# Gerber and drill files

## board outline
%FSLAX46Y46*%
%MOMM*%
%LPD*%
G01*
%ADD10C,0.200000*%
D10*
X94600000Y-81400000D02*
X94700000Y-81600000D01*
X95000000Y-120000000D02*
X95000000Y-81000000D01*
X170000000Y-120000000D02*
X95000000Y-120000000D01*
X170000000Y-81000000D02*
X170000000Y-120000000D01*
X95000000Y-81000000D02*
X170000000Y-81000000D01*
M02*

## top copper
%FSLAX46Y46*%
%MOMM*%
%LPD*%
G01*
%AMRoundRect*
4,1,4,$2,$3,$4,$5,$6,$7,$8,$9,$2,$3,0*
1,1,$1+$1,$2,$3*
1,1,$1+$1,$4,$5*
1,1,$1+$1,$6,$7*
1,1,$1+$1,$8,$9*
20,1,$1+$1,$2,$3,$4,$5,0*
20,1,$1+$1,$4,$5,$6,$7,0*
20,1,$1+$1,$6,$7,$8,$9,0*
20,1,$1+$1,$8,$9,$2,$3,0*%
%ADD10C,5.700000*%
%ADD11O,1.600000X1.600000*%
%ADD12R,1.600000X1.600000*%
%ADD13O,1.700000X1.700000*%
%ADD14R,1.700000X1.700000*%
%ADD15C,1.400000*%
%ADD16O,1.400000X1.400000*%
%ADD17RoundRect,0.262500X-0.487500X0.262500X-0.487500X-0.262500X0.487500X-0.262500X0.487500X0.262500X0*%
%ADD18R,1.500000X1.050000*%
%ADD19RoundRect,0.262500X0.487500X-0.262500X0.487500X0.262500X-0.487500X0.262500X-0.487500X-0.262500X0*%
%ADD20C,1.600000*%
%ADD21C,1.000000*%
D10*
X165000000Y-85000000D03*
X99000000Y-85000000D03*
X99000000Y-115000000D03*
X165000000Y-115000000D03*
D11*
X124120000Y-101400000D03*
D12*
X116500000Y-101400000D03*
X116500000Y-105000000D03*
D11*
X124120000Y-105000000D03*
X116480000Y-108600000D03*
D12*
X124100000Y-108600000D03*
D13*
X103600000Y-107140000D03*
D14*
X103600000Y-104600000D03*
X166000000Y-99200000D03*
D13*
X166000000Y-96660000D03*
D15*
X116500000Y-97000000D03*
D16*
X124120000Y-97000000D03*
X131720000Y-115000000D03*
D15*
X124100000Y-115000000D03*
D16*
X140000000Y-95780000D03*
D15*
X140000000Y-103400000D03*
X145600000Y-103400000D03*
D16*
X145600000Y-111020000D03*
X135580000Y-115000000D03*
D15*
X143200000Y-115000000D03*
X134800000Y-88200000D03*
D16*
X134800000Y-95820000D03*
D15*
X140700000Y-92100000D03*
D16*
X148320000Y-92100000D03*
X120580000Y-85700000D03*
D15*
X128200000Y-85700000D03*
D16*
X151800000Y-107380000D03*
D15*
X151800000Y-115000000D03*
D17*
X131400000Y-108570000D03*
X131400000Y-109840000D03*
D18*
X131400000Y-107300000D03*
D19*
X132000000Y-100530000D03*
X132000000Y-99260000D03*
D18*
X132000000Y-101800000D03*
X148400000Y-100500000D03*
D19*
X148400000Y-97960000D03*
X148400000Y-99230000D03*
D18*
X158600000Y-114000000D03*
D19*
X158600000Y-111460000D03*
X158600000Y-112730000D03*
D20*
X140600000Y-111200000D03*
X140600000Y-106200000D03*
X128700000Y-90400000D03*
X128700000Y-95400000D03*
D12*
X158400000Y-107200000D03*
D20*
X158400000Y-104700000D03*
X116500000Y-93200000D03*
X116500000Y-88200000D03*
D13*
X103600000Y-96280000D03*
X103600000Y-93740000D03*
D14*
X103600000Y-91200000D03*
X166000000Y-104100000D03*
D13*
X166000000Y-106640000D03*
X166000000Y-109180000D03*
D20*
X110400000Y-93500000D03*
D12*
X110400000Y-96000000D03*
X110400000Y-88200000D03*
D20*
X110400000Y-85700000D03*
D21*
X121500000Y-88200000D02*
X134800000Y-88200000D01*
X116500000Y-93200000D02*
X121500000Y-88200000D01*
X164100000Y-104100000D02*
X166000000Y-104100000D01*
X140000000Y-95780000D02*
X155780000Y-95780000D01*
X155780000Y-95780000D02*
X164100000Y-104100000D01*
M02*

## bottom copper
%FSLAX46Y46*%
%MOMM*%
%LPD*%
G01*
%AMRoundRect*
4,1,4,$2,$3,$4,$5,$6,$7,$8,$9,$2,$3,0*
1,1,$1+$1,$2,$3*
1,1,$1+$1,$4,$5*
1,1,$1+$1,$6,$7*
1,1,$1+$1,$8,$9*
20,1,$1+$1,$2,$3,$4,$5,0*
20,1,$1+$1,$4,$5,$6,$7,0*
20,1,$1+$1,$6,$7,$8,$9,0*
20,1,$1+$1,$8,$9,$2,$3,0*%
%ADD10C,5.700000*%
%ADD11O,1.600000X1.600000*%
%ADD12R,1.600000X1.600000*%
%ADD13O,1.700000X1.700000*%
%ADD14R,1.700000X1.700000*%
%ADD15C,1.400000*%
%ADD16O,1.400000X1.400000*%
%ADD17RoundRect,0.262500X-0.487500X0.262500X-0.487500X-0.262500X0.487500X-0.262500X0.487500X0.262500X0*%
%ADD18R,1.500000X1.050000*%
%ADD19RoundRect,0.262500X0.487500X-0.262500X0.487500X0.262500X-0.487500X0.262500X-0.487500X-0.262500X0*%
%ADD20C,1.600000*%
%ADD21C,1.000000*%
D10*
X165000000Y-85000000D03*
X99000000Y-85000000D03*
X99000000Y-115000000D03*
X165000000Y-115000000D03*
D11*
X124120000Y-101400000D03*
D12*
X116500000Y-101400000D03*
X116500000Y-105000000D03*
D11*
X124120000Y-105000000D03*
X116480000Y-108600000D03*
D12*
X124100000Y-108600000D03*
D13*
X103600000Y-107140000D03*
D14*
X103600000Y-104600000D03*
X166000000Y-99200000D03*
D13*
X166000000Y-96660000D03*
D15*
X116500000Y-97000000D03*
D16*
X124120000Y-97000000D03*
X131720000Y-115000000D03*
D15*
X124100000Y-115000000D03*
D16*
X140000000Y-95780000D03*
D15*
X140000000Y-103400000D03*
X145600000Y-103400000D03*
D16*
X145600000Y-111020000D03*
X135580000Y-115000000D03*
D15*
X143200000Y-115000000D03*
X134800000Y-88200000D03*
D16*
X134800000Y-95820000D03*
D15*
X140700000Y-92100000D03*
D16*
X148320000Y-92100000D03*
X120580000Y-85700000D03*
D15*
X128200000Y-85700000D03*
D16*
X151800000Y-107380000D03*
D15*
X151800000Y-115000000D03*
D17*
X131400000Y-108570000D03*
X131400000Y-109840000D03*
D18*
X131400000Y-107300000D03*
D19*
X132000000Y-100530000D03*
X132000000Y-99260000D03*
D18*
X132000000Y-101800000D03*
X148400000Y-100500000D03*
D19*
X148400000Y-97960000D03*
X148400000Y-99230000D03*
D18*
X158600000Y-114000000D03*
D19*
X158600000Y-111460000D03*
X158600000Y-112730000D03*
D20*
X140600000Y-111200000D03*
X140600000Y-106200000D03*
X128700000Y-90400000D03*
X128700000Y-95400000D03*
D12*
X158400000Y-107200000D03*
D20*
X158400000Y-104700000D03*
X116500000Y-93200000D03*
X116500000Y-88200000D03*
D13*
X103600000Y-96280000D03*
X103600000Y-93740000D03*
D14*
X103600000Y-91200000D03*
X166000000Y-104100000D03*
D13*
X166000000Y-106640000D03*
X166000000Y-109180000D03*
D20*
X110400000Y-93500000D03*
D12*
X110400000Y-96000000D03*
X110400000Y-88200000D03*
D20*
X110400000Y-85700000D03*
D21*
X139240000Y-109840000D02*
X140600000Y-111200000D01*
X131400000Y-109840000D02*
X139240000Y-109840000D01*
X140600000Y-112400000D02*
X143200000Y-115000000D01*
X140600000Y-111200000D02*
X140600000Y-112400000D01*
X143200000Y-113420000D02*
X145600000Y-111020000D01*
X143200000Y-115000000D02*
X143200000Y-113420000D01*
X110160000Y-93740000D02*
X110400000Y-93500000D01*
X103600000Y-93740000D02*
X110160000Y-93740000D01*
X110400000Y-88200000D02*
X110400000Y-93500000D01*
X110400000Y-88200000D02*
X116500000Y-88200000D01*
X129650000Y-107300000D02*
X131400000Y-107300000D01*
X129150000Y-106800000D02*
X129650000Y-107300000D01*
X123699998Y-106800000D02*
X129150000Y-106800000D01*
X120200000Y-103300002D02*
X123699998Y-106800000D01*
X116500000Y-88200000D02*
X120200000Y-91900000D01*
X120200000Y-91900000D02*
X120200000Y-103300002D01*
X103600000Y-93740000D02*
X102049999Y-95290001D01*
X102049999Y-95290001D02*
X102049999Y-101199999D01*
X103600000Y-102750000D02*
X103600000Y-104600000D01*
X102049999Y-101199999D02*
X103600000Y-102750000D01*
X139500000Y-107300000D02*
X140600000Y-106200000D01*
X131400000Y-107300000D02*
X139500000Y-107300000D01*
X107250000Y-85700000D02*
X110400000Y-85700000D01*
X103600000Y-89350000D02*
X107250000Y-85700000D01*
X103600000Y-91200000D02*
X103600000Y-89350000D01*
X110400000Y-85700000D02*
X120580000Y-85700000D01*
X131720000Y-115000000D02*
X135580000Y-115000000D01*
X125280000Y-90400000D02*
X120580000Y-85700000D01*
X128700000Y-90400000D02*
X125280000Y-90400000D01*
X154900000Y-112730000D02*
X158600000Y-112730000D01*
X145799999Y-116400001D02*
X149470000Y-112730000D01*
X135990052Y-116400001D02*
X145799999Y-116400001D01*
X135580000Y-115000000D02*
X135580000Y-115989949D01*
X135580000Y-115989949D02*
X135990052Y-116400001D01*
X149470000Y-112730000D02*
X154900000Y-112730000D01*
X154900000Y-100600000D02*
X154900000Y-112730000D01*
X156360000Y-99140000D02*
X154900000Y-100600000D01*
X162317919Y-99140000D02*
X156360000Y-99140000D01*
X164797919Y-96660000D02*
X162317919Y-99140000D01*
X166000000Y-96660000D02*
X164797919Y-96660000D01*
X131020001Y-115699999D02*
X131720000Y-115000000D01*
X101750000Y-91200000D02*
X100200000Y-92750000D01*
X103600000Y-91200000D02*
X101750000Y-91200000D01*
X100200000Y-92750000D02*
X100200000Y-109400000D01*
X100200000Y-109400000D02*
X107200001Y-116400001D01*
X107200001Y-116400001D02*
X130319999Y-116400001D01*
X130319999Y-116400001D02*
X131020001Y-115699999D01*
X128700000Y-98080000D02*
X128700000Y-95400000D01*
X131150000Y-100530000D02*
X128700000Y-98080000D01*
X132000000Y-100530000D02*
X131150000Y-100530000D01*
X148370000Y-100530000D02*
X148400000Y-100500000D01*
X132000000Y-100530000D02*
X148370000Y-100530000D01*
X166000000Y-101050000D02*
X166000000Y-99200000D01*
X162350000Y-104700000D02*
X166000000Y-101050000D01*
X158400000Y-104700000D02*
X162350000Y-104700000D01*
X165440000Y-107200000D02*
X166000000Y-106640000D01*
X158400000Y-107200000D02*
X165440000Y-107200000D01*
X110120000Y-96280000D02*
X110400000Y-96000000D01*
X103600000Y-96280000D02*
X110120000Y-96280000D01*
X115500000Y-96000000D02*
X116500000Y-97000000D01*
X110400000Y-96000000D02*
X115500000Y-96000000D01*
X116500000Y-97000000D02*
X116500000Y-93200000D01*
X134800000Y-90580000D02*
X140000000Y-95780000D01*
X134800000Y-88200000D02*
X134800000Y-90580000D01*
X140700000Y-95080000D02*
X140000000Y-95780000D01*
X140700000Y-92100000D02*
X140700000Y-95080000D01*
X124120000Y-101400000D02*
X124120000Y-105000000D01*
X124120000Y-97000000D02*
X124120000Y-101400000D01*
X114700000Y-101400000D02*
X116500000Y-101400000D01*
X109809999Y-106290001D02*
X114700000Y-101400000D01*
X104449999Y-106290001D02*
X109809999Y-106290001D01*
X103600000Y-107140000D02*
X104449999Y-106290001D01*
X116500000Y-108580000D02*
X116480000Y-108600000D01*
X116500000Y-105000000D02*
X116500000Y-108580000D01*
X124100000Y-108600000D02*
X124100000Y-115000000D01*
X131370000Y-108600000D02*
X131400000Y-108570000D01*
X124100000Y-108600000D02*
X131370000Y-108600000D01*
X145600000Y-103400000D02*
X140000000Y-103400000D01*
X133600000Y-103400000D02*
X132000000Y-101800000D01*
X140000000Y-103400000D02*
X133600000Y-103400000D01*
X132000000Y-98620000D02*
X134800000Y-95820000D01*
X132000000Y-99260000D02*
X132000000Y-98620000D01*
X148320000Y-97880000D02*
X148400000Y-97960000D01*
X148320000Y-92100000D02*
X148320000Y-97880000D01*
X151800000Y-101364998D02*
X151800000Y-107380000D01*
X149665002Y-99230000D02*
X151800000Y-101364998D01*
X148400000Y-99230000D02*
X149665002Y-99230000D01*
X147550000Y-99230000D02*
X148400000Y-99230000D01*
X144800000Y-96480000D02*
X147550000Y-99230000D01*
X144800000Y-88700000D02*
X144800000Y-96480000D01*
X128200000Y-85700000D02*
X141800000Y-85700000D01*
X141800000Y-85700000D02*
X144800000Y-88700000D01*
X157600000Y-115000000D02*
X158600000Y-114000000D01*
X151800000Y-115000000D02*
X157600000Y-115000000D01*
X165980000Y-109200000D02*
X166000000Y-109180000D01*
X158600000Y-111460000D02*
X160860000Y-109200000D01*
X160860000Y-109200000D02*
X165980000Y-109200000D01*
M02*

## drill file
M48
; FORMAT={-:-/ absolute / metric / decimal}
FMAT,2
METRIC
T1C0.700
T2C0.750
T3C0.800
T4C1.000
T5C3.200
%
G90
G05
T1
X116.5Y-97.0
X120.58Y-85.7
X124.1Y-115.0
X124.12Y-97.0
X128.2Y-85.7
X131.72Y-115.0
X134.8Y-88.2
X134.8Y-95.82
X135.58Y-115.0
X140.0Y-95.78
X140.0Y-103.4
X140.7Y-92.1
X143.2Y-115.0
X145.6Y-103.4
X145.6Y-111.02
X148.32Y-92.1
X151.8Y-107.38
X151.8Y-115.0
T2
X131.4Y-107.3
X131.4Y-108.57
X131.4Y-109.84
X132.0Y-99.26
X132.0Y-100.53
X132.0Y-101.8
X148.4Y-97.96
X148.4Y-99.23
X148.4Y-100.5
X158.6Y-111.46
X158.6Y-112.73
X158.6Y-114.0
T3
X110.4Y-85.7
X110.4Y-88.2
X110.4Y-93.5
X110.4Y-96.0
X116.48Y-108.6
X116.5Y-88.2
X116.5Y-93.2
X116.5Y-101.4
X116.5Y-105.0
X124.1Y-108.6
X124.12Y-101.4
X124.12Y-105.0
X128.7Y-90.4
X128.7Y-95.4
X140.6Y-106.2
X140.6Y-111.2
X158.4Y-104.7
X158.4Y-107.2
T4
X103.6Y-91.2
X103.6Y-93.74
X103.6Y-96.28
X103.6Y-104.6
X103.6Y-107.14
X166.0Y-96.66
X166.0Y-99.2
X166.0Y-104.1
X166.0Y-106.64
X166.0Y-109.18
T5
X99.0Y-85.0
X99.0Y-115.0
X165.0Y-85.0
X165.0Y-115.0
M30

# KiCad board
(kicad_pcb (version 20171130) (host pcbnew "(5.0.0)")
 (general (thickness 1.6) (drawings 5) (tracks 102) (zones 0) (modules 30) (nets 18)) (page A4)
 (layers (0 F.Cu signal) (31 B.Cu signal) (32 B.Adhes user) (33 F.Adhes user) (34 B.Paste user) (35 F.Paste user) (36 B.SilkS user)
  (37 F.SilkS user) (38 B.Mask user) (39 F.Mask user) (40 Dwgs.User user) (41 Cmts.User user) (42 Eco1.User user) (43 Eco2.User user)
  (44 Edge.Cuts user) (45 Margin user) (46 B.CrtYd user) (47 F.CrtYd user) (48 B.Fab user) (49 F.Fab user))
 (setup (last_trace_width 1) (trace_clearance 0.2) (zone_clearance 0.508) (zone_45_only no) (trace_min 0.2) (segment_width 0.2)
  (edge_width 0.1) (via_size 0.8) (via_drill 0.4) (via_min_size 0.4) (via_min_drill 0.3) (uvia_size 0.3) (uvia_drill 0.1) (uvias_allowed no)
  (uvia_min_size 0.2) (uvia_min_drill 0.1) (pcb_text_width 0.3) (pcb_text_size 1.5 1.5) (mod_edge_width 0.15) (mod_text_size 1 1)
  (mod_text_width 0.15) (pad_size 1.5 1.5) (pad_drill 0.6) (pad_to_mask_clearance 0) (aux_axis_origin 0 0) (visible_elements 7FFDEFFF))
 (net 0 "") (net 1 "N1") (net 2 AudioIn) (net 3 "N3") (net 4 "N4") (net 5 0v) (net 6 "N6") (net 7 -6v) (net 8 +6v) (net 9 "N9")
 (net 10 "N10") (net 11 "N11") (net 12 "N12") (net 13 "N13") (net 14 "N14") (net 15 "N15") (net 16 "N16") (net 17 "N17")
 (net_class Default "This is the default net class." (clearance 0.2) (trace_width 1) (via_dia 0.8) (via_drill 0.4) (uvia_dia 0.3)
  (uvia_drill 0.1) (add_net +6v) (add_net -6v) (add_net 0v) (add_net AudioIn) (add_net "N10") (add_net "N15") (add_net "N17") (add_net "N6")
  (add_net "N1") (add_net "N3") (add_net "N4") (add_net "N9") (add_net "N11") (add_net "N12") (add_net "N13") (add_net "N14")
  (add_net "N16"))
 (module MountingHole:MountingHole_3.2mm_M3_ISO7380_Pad (layer F.Cu) (at 165 85)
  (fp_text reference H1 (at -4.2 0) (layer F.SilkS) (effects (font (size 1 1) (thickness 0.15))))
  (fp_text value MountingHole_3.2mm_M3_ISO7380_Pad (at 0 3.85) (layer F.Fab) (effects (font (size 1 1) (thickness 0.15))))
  (pad 1 thru_hole circle (at 0 0) (size 5.7 5.7) (drill 3.2) (layers *.Cu *.Mask)))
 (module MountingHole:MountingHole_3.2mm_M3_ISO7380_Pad (layer F.Cu) (at 99 85)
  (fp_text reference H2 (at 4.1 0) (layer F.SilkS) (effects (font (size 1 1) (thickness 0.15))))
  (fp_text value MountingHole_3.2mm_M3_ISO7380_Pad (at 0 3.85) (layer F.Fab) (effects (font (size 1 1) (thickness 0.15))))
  (pad 1 thru_hole circle (at 0 0) (size 5.7 5.7) (drill 3.2) (layers *.Cu *.Mask)))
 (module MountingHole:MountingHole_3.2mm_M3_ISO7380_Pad (layer F.Cu) (at 99 115)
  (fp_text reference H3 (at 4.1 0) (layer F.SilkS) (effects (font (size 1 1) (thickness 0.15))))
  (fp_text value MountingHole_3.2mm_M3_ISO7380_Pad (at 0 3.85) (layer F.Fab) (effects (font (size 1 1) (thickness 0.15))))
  (pad 1 thru_hole circle (at 0 0) (size 5.7 5.7) (drill 3.2) (layers *.Cu *.Mask)))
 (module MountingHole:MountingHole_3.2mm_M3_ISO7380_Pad (layer F.Cu) (at 165 115)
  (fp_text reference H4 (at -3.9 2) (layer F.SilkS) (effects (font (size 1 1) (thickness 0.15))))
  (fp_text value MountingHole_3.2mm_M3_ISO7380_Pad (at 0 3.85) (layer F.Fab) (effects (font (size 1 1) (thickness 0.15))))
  (pad 1 thru_hole circle (at 0 0) (size 5.7 5.7) (drill 3.2) (layers *.Cu *.Mask)))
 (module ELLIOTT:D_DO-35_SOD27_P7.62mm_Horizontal (layer F.Cu) (at 116.5 101.4)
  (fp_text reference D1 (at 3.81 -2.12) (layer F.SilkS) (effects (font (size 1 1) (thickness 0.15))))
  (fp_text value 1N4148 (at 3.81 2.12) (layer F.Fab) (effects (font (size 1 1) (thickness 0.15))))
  (pad 2 thru_hole oval (at 7.62 0) (size 1.6 1.6) (drill 0.8) (layers *.Cu *.Mask) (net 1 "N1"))
  (pad 1 thru_hole rect (at 0 0) (size 1.6 1.6) (drill 0.8) (layers *.Cu *.Mask) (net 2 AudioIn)))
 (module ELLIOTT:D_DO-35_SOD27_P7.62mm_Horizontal (layer F.Cu) (at 116.5 105)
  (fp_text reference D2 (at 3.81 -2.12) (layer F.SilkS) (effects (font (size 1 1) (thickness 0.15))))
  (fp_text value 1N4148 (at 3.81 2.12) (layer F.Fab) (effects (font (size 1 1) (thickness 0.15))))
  (pad 1 thru_hole rect (at 0 0) (size 1.6 1.6) (drill 0.8) (layers *.Cu *.Mask) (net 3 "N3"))
  (pad 2 thru_hole oval (at 7.62 0) (size 1.6 1.6) (drill 0.8) (layers *.Cu *.Mask) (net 1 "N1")))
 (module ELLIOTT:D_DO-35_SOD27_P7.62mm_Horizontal (layer F.Cu) (at 124.1 108.6 180)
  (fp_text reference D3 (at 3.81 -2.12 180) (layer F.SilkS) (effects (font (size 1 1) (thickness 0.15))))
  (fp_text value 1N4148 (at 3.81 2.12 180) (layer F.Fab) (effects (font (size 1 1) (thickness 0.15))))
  (pad 2 thru_hole oval (at 7.62 0 180) (size 1.6 1.6) (drill 0.8) (layers *.Cu *.Mask) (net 3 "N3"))
  (pad 1 thru_hole rect (at 0 0 180) (size 1.6 1.6) (drill 0.8) (layers *.Cu *.Mask) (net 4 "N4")))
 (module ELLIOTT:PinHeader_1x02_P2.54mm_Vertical (layer F.Cu) (at 103.6 104.6)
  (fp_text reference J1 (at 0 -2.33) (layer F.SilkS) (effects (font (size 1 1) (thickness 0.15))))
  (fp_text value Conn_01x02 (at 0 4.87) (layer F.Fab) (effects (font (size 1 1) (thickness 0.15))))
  (pad 2 thru_hole oval (at 0 2.54) (size 1.7 1.7) (drill 1) (layers *.Cu *.Mask) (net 2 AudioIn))
  (pad 1 thru_hole rect (at 0 0) (size 1.7 1.7) (drill 1) (layers *.Cu *.Mask) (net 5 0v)))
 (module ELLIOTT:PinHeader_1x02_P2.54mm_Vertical (layer F.Cu) (at 166 99.2 180)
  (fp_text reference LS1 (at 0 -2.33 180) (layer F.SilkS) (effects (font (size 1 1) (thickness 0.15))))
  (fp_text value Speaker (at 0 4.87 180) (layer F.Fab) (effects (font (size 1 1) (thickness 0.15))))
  (pad 1 thru_hole rect (at 0 0 180) (size 1.7 1.7) (drill 1) (layers *.Cu *.Mask) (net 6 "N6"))
  (pad 2 thru_hole oval (at 0 2.54 180) (size 1.7 1.7) (drill 1) (layers *.Cu *.Mask) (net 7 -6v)))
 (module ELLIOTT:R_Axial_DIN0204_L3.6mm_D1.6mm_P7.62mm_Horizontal (layer F.Cu) (at 116.5 97)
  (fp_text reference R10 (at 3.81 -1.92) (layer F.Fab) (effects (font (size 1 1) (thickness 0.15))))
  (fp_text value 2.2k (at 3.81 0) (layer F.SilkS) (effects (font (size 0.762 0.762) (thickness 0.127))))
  (pad 1 thru_hole circle (at 0 0) (size 1.4 1.4) (drill 0.7) (layers *.Cu *.Mask) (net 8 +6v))
  (pad 2 thru_hole oval (at 7.62 0) (size 1.4 1.4) (drill 0.7) (layers *.Cu *.Mask) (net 1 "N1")))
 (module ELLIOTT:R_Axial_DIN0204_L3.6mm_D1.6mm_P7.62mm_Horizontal (layer F.Cu) (at 124.1 115)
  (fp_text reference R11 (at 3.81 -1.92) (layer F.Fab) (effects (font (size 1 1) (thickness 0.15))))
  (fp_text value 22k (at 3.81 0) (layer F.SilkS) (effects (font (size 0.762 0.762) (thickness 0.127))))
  (pad 2 thru_hole oval (at 7.62 0) (size 1.4 1.4) (drill 0.7) (layers *.Cu *.Mask) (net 7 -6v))
  (pad 1 thru_hole circle (at 0 0) (size 1.4 1.4) (drill 0.7) (layers *.Cu *.Mask) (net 4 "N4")))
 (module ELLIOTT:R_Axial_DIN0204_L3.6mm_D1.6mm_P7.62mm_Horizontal (layer F.Cu) (at 140 103.4 90)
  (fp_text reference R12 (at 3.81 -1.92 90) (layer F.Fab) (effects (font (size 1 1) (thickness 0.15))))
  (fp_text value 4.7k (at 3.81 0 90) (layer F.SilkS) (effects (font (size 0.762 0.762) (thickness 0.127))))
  (pad 2 thru_hole oval (at 7.62 0 90) (size 1.4 1.4) (drill 0.7) (layers *.Cu *.Mask) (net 8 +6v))
  (pad 1 thru_hole circle (at 0 0 90) (size 1.4 1.4) (drill 0.7) (layers *.Cu *.Mask) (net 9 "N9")))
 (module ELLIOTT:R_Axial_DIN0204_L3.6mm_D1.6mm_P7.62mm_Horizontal (layer F.Cu) (at 145.6 103.4 270)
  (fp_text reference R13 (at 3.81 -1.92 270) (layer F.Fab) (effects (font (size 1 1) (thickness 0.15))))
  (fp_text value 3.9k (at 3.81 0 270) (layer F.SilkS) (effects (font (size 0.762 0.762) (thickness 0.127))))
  (pad 1 thru_hole circle (at 0 0 270) (size 1.4 1.4) (drill 0.7) (layers *.Cu *.Mask) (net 9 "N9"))
  (pad 2 thru_hole oval (at 7.62 0 270) (size 1.4 1.4) (drill 0.7) (layers *.Cu *.Mask) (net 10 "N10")))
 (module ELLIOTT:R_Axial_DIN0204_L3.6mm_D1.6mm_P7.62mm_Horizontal (layer F.Cu) (at 143.2 115 180)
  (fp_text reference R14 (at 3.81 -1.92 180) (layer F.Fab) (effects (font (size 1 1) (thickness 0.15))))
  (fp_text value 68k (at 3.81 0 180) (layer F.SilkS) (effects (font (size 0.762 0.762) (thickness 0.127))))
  (pad 2 thru_hole oval (at 7.62 0 180) (size 1.4 1.4) (drill 0.7) (layers *.Cu *.Mask) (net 7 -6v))
  (pad 1 thru_hole circle (at 0 0 180) (size 1.4 1.4) (drill 0.7) (layers *.Cu *.Mask) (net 10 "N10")))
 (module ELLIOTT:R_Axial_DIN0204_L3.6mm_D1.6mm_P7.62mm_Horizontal (layer F.Cu) (at 134.8 88.2 270)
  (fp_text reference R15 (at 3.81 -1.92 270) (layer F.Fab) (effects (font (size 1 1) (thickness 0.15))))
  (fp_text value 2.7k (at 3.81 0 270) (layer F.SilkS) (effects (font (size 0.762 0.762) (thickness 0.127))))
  (pad 1 thru_hole circle (at 0 0 270) (size 1.4 1.4) (drill 0.7) (layers *.Cu *.Mask) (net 8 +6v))
  (pad 2 thru_hole oval (at 7.62 0 270) (size 1.4 1.4) (drill 0.7) (layers *.Cu *.Mask) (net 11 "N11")))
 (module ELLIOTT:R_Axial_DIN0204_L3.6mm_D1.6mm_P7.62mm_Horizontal (layer F.Cu) (at 140.7 92.1)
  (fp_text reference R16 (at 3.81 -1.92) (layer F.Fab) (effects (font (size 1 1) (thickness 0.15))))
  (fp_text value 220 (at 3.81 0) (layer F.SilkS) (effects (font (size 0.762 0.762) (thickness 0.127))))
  (pad 1 thru_hole circle (at 0 0) (size 1.4 1.4) (drill 0.7) (layers *.Cu *.Mask) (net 8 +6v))
  (pad 2 thru_hole oval (at 7.62 0) (size 1.4 1.4) (drill 0.7) (layers *.Cu *.Mask) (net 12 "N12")))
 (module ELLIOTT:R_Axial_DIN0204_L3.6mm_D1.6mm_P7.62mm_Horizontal (layer F.Cu) (at 128.2 85.7 180)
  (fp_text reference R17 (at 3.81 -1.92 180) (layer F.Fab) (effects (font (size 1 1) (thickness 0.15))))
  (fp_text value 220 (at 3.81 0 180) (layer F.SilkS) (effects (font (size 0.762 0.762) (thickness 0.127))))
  (pad 2 thru_hole oval (at 7.62 0 180) (size 1.4 1.4) (drill 0.7) (layers *.Cu *.Mask) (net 7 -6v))
  (pad 1 thru_hole circle (at 0 0 180) (size 1.4 1.4) (drill 0.7) (layers *.Cu *.Mask) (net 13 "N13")))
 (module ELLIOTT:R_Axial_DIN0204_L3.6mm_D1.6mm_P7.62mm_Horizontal (layer F.Cu) (at 151.8 115 90)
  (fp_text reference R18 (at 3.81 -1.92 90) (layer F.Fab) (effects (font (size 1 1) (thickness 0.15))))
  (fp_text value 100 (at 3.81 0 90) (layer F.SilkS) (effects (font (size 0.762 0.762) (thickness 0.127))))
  (pad 2 thru_hole oval (at 7.62 0 90) (size 1.4 1.4) (drill 0.7) (layers *.Cu *.Mask) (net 13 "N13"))
  (pad 1 thru_hole circle (at 0 0 90) (size 1.4 1.4) (drill 0.7) (layers *.Cu *.Mask) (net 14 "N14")))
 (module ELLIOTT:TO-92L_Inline (layer F.Cu) (at 131.4 107.3 270)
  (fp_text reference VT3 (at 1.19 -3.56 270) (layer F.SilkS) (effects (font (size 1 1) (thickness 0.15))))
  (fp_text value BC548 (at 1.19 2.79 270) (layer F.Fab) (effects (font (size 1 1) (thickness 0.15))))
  (pad 2 thru_hole roundrect (at 1.27 0 270) (size 1.05 1.5) (drill 0.75) (layers *.Cu *.Mask) (roundrect_rratio 0.25) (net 4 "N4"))
  (pad 3 thru_hole roundrect (at 2.54 0 270) (size 1.05 1.5) (drill 0.75) (layers *.Cu *.Mask) (roundrect_rratio 0.25) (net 10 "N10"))
  (pad 1 thru_hole rect (at 0 0 270) (size 1.05 1.5) (drill 0.75) (layers *.Cu *.Mask) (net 5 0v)))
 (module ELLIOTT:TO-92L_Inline (layer F.Cu) (at 132 101.8 90)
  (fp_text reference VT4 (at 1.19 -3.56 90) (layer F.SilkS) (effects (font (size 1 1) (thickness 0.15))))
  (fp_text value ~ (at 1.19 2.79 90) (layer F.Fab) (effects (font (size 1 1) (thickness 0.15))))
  (pad 2 thru_hole roundrect (at 1.27 0 90) (size 1.05 1.5) (drill 0.75) (layers *.Cu *.Mask) (roundrect_rratio 0.25) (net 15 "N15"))
  (pad 3 thru_hole roundrect (at 2.54 0 90) (size 1.05 1.5) (drill 0.75) (layers *.Cu *.Mask) (roundrect_rratio 0.25) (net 11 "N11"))
  (pad 1 thru_hole rect (at 0 0 90) (size 1.05 1.5) (drill 0.75) (layers *.Cu *.Mask) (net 9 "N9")))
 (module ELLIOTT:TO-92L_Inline (layer F.Cu) (at 148.4 100.5 90)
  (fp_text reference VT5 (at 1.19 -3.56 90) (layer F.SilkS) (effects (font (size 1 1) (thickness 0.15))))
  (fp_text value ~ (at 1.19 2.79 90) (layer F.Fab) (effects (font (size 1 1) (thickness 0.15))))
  (pad 1 thru_hole rect (at 0 0 90) (size 1.05 1.5) (drill 0.75) (layers *.Cu *.Mask) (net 15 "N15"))
  (pad 3 thru_hole roundrect (at 2.54 0 90) (size 1.05 1.5) (drill 0.75) (layers *.Cu *.Mask) (roundrect_rratio 0.25) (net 12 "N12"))
  (pad 2 thru_hole roundrect (at 1.27 0 90) (size 1.05 1.5) (drill 0.75) (layers *.Cu *.Mask) (roundrect_rratio 0.25) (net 13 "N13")))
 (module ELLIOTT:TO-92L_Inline (layer F.Cu) (at 158.6 114 90)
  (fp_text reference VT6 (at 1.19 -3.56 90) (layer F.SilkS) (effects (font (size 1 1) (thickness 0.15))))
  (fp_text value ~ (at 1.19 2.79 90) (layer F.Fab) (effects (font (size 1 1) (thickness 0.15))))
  (pad 1 thru_hole rect (at 0 0 90) (size 1.05 1.5) (drill 0.75) (layers *.Cu *.Mask) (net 14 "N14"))
  (pad 3 thru_hole roundrect (at 2.54 0 90) (size 1.05 1.5) (drill 0.75) (layers *.Cu *.Mask) (roundrect_rratio 0.25) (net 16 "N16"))
  (pad 2 thru_hole roundrect (at 1.27 0 90) (size 1.05 1.5) (drill 0.75) (layers *.Cu *.Mask) (roundrect_rratio 0.25) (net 7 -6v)))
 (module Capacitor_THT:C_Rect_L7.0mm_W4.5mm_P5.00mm (layer F.Cu) (at 140.6 111.2 90)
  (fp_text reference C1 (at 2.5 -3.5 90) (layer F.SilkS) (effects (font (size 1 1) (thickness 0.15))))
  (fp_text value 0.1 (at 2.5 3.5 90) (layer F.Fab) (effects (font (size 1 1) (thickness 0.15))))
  (pad 1 thru_hole circle (at 0 0 90) (size 1.6 1.6) (drill 0.8) (layers *.Cu *.Mask) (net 10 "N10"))
  (pad 2 thru_hole circle (at 5 0 90) (size 1.6 1.6) (drill 0.8) (layers *.Cu *.Mask) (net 5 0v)))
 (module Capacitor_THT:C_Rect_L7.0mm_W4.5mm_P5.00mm (layer F.Cu) (at 128.7 95.4 90)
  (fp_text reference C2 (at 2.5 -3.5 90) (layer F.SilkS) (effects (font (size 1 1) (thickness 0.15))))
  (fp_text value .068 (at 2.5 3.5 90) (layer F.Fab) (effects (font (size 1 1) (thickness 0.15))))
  (pad 2 thru_hole circle (at 5 0 90) (size 1.6 1.6) (drill 0.8) (layers *.Cu *.Mask) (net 7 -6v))
  (pad 1 thru_hole circle (at 0 0 90) (size 1.6 1.6) (drill 0.8) (layers *.Cu *.Mask) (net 15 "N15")))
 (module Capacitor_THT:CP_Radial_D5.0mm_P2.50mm (layer F.Cu) (at 158.4 107.2 90)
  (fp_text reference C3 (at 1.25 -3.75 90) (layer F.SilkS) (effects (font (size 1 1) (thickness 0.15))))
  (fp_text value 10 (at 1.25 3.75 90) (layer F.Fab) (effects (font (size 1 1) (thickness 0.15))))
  (pad 1 thru_hole rect (at 0 0 90) (size 1.6 1.6) (drill 0.8) (layers *.Cu *.Mask) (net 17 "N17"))
  (pad 2 thru_hole circle (at 2.5 0 90) (size 1.6 1.6) (drill 0.8) (layers *.Cu *.Mask) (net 6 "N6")))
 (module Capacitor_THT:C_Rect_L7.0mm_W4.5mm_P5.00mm (layer F.Cu) (at 116.5 93.2 90)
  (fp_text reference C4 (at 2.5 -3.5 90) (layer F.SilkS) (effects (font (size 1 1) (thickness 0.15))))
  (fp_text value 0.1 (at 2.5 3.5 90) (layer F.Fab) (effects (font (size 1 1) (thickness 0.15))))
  (pad 1 thru_hole circle (at 0 0 90) (size 1.6 1.6) (drill 0.8) (layers *.Cu *.Mask) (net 8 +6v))
  (pad 2 thru_hole circle (at 5 0 90) (size 1.6 1.6) (drill 0.8) (layers *.Cu *.Mask) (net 5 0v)))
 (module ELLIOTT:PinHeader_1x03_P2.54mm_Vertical (layer F.Cu) (at 103.6 91.2)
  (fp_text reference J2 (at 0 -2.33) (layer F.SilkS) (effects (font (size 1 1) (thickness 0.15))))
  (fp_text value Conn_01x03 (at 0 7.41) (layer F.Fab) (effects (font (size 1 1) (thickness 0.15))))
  (pad 3 thru_hole oval (at 0 5.08) (size 1.7 1.7) (drill 1) (layers *.Cu *.Mask) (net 8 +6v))
  (pad 2 thru_hole oval (at 0 2.54) (size 1.7 1.7) (drill 1) (layers *.Cu *.Mask) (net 5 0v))
  (pad 1 thru_hole rect (at 0 0) (size 1.7 1.7) (drill 1) (layers *.Cu *.Mask) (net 7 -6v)))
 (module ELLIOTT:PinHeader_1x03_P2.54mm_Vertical (layer F.Cu) (at 166 104.1)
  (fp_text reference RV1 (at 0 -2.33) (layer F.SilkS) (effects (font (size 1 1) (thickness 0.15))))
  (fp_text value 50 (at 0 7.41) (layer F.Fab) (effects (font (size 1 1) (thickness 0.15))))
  (pad 1 thru_hole rect (at 0 0) (size 1.7 1.7) (drill 1) (layers *.Cu *.Mask) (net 8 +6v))
  (pad 2 thru_hole oval (at 0 2.54) (size 1.7 1.7) (drill 1) (layers *.Cu *.Mask) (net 17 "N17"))
  (pad 3 thru_hole oval (at 0 5.08) (size 1.7 1.7) (drill 1) (layers *.Cu *.Mask) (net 16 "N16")))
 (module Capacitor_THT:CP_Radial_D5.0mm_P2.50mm (layer F.Cu) (at 110.4 96 90)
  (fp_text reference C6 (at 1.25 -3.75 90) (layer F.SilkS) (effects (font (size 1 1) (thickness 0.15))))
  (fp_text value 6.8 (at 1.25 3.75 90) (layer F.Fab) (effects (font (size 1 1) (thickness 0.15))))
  (pad 2 thru_hole circle (at 2.5 0 90) (size 1.6 1.6) (drill 0.8) (layers *.Cu *.Mask) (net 5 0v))
  (pad 1 thru_hole rect (at 0 0 90) (size 1.6 1.6) (drill 0.8) (layers *.Cu *.Mask) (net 8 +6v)))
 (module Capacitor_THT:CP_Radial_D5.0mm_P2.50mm (layer F.Cu) (at 110.4 88.2 90)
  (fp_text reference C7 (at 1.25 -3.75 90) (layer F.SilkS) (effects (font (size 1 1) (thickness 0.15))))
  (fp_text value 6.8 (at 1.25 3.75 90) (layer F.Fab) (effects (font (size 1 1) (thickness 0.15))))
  (pad 1 thru_hole rect (at 0 0 90) (size 1.6 1.6) (drill 0.8) (layers *.Cu *.Mask) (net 5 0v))
  (pad 2 thru_hole circle (at 2.5 0 90) (size 1.6 1.6) (drill 0.8) (layers *.Cu *.Mask) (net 7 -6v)))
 (gr_line (start 94.6 81.4) (end 94.7 81.6) (layer Edge.Cuts) (width 0.2))
 (gr_line (start 95 120) (end 95 81) (layer Edge.Cuts) (width 0.2))
 (gr_line (start 170 120) (end 95 120) (layer Edge.Cuts) (width 0.2))
 (gr_line (start 170 81) (end 170 120) (layer Edge.Cuts) (width 0.2))
 (gr_line (start 95 81) (end 170 81) (layer Edge.Cuts) (width 0.2))
 (segment (start 139.24 109.84) (end 140.6 111.2) (width 1) (layer B.Cu) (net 10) (status 20))
 (segment (start 131.4 109.84) (end 139.24 109.84) (width 1) (layer B.Cu) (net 10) (status 10))
 (segment (start 140.6 112.4) (end 143.2 115) (width 1) (layer B.Cu) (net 10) (status 20))
 (segment (start 140.6 111.2) (end 140.6 112.4) (width 1) (layer B.Cu) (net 10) (status 10))
 (segment (start 143.2 113.42) (end 145.6 111.02) (width 1) (layer B.Cu) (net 10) (status 20))
 (segment (start 143.2 115) (end 143.2 113.42) (width 1) (layer B.Cu) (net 10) (status 10))
 (segment (start 110.16 93.74) (end 110.4 93.5) (width 1) (layer B.Cu) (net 5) (status 30))
 (segment (start 103.6 93.74) (end 110.16 93.74) (width 1) (layer B.Cu) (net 5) (status 30))
 (segment (start 110.4 88.2) (end 110.4 93.5) (width 1) (layer B.Cu) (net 5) (status 30))
 (segment (start 110.4 88.2) (end 116.5 88.2) (width 1) (layer B.Cu) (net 5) (status 30))
 (segment (start 129.65 107.3) (end 131.4 107.3) (width 1) (layer B.Cu) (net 5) (status 20))
 (segment (start 129.15 106.8) (end 129.65 107.3) (width 1) (layer B.Cu) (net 5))
 (segment (start 123.699998 106.8) (end 129.15 106.8) (width 1) (layer B.Cu) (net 5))
 (segment (start 120.2 103.300002) (end 123.699998 106.8) (width 1) (layer B.Cu) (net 5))
 (segment (start 116.5 88.2) (end 120.2 91.9) (width 1) (layer B.Cu) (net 5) (status 10))
 (segment (start 120.2 91.9) (end 120.2 103.300002) (width 1) (layer B.Cu) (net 5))
 (segment (start 103.6 93.74) (end 102.049999 95.290001) (width 1) (layer B.Cu) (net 5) (status 10))
 (segment (start 102.049999 95.290001) (end 102.049999 101.199999) (width 1) (layer B.Cu) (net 5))
 (segment (start 103.6 102.75) (end 103.6 104.6) (width 1) (layer B.Cu) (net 5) (status 20))
 (segment (start 102.049999 101.199999) (end 103.6 102.75) (width 1) (layer B.Cu) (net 5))
 (segment (start 139.5 107.3) (end 140.6 106.2) (width 1) (layer B.Cu) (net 5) (status 20))
 (segment (start 131.4 107.3) (end 139.5 107.3) (width 1) (layer B.Cu) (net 5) (status 10))
 (segment (start 107.25 85.7) (end 110.4 85.7) (width 1) (layer B.Cu) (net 7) (status 20))
 (segment (start 103.6 89.35) (end 107.25 85.7) (width 1) (layer B.Cu) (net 7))
 (segment (start 103.6 91.2) (end 103.6 89.35) (width 1) (layer B.Cu) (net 7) (status 10))
 (segment (start 110.4 85.7) (end 120.58 85.7) (width 1) (layer B.Cu) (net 7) (status 30))
 (segment (start 131.72 115) (end 135.58 115) (width 1) (layer B.Cu) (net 7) (status 30))
 (segment (start 125.28 90.4) (end 120.58 85.7) (width 1) (layer B.Cu) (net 7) (status 20))
 (segment (start 128.7 90.4) (end 125.28 90.4) (width 1) (layer B.Cu) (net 7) (status 10))
 (segment (start 154.9 112.73) (end 158.6 112.73) (width 1) (layer B.Cu) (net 7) (status 20))
 (segment (start 145.799999 116.400001) (end 149.47 112.73) (width 1) (layer B.Cu) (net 7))
 (segment (start 135.990052 116.400001) (end 145.799999 116.400001) (width 1) (layer B.Cu) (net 7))
 (segment (start 135.58 115) (end 135.58 115.989949) (width 1) (layer B.Cu) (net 7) (status 10))
 (segment (start 135.58 115.989949) (end 135.990052 116.400001) (width 1) (layer B.Cu) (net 7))
 (segment (start 149.47 112.73) (end 154.9 112.73) (width 1) (layer B.Cu) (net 7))
 (segment (start 154.9 100.6) (end 154.9 112.73) (width 1) (layer B.Cu) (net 7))
 (segment (start 156.36 99.14) (end 154.9 100.6) (width 1) (layer B.Cu) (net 7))
 (segment (start 162.317919 99.14) (end 156.36 99.14) (width 1) (layer B.Cu) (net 7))
 (segment (start 164.797919 96.66) (end 162.317919 99.14) (width 1) (layer B.Cu) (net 7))
 (segment (start 166 96.66) (end 164.797919 96.66) (width 1) (layer B.Cu) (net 7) (status 10))
 (segment (start 131.020001 115.699999) (end 131.72 115) (width 1) (layer B.Cu) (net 7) (status 30))
 (segment (start 101.75 91.2) (end 100.2 92.75) (width 1) (layer B.Cu) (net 7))
 (segment (start 103.6 91.2) (end 101.75 91.2) (width 1) (layer B.Cu) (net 7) (status 10))
 (segment (start 100.2 92.75) (end 100.2 109.4) (width 1) (layer B.Cu) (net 7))
 (segment (start 100.2 109.4) (end 107.200001 116.400001) (width 1) (layer B.Cu) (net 7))
 (segment (start 107.200001 116.400001) (end 130.319999 116.400001) (width 1) (layer B.Cu) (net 7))
 (segment (start 130.319999 116.400001) (end 131.020001 115.699999) (width 1) (layer B.Cu) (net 7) (status 20))
 (segment (start 128.7 98.08) (end 128.7 95.4) (width 1) (layer B.Cu) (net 15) (status 20))
 (segment (start 131.15 100.53) (end 128.7 98.08) (width 1) (layer B.Cu) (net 15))
 (segment (start 132 100.53) (end 131.15 100.53) (width 1) (layer B.Cu) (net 15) (status 10))
 (segment (start 148.37 100.53) (end 148.4 100.5) (width 1) (layer B.Cu) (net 15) (status 30))
 (segment (start 132 100.53) (end 148.37 100.53) (width 1) (layer B.Cu) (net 15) (status 30))
 (segment (start 166 101.05) (end 166 99.2) (width 1) (layer B.Cu) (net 6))
 (segment (start 162.35 104.7) (end 166 101.05) (width 1) (layer B.Cu) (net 6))
 (segment (start 158.4 104.7) (end 162.35 104.7) (width 1) (layer B.Cu) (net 6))
 (segment (start 165.44 107.2) (end 166 106.64) (width 1) (layer B.Cu) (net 17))
 (segment (start 158.4 107.2) (end 165.44 107.2) (width 1) (layer B.Cu) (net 17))
 (segment (start 110.12 96.28) (end 110.4 96) (width 1) (layer B.Cu) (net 8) (status 30))
 (segment (start 103.6 96.28) (end 110.12 96.28) (width 1) (layer B.Cu) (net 8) (status 30))
 (segment (start 115.5 96) (end 116.5 97) (width 1) (layer B.Cu) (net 8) (status 20))
 (segment (start 110.4 96) (end 115.5 96) (width 1) (layer B.Cu) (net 8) (status 10))
 (segment (start 116.5 97) (end 116.5 93.2) (width 1) (layer B.Cu) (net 8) (status 30))
 (segment (start 121.5 88.2) (end 134.8 88.2) (width 1) (layer F.Cu) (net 8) (status 20))
 (segment (start 116.5 93.2) (end 121.5 88.2) (width 1) (layer F.Cu) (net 8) (status 10))
 (segment (start 134.8 90.58) (end 140 95.78) (width 1) (layer B.Cu) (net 8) (status 20))
 (segment (start 134.8 88.2) (end 134.8 90.58) (width 1) (layer B.Cu) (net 8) (status 10))
 (segment (start 140.7 95.08) (end 140 95.78) (width 1) (layer B.Cu) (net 8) (status 30))
 (segment (start 140.7 92.1) (end 140.7 95.08) (width 1) (layer B.Cu) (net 8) (status 30))
 (segment (start 164.1 104.1) (end 166 104.1) (width 1) (layer F.Cu) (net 8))
 (segment (start 140 95.78) (end 155.78 95.78) (width 1) (layer F.Cu) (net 8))
 (segment (start 155.78 95.78) (end 164.1 104.1) (width 1) (layer F.Cu) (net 8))
 (segment (start 124.12 101.4) (end 124.12 105) (width 1) (layer B.Cu) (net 1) (status 30))
 (segment (start 124.12 97) (end 124.12 101.4) (width 1) (layer B.Cu) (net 1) (status 30))
 (segment (start 114.7 101.4) (end 116.5 101.4) (width 1) (layer B.Cu) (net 2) (status 20))
 (segment (start 109.809999 106.290001) (end 114.7 101.4) (width 1) (layer B.Cu) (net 2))
 (segment (start 104.449999 106.290001) (end 109.809999 106.290001) (width 1) (layer B.Cu) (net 2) (status 10))
 (segment (start 103.6 107.14) (end 104.449999 106.290001) (width 1) (layer B.Cu) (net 2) (status 30))
 (segment (start 116.5 108.58) (end 116.48 108.6) (width 1) (layer B.Cu) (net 3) (status 30))
 (segment (start 116.5 105) (end 116.5 108.58) (width 1) (layer B.Cu) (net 3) (status 30))
 (segment (start 124.1 108.6) (end 124.1 115) (width 1) (layer B.Cu) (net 4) (status 30))
 (segment (start 131.37 108.6) (end 131.4 108.57) (width 1) (layer B.Cu) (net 4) (status 30))
 (segment (start 124.1 108.6) (end 131.37 108.6) (width 1) (layer B.Cu) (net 4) (status 30))
 (segment (start 145.6 103.4) (end 140 103.4) (width 1) (layer B.Cu) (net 9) (status 30))
 (segment (start 133.6 103.4) (end 132 101.8) (width 1) (layer B.Cu) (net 9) (status 20))
 (segment (start 140 103.4) (end 133.6 103.4) (width 1) (layer B.Cu) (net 9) (status 10))
 (segment (start 132 98.62) (end 134.8 95.82) (width 1) (layer B.Cu) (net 11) (status 20))
 (segment (start 132 99.26) (end 132 98.62) (width 1) (layer B.Cu) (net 11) (status 10))
 (segment (start 148.32 97.88) (end 148.4 97.96) (width 1) (layer B.Cu) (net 12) (status 30))
 (segment (start 148.32 92.1) (end 148.32 97.88) (width 1) (layer B.Cu) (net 12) (status 30))
 (segment (start 151.8 101.364998) (end 151.8 107.38) (width 1) (layer B.Cu) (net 13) (status 20))
 (segment (start 149.665002 99.23) (end 151.8 101.364998) (width 1) (layer B.Cu) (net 13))
 (segment (start 148.4 99.23) (end 149.665002 99.23) (width 1) (layer B.Cu) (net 13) (status 10))
 (segment (start 147.55 99.23) (end 148.4 99.23) (width 1) (layer B.Cu) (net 13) (status 20))
 (segment (start 144.8 96.48) (end 147.55 99.23) (width 1) (layer B.Cu) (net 13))
 (segment (start 144.8 88.7) (end 144.8 96.48) (width 1) (layer B.Cu) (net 13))
 (segment (start 128.2 85.7) (end 141.8 85.7) (width 1) (layer B.Cu) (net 13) (status 10))
 (segment (start 141.8 85.7) (end 144.8 88.7) (width 1) (layer B.Cu) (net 13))
 (segment (start 157.6 115) (end 158.6 114) (width 1) (layer B.Cu) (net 14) (status 20))
 (segment (start 151.8 115) (end 157.6 115) (width 1) (layer B.Cu) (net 14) (status 10))
 (segment (start 165.98 109.2) (end 166 109.18) (width 1) (layer B.Cu) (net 16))
 (segment (start 158.6 111.46) (end 160.86 109.2) (width 1) (layer B.Cu) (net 16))
 (segment (start 160.86 109.2) (end 165.98 109.2) (width 1) (layer B.Cu) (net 16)))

